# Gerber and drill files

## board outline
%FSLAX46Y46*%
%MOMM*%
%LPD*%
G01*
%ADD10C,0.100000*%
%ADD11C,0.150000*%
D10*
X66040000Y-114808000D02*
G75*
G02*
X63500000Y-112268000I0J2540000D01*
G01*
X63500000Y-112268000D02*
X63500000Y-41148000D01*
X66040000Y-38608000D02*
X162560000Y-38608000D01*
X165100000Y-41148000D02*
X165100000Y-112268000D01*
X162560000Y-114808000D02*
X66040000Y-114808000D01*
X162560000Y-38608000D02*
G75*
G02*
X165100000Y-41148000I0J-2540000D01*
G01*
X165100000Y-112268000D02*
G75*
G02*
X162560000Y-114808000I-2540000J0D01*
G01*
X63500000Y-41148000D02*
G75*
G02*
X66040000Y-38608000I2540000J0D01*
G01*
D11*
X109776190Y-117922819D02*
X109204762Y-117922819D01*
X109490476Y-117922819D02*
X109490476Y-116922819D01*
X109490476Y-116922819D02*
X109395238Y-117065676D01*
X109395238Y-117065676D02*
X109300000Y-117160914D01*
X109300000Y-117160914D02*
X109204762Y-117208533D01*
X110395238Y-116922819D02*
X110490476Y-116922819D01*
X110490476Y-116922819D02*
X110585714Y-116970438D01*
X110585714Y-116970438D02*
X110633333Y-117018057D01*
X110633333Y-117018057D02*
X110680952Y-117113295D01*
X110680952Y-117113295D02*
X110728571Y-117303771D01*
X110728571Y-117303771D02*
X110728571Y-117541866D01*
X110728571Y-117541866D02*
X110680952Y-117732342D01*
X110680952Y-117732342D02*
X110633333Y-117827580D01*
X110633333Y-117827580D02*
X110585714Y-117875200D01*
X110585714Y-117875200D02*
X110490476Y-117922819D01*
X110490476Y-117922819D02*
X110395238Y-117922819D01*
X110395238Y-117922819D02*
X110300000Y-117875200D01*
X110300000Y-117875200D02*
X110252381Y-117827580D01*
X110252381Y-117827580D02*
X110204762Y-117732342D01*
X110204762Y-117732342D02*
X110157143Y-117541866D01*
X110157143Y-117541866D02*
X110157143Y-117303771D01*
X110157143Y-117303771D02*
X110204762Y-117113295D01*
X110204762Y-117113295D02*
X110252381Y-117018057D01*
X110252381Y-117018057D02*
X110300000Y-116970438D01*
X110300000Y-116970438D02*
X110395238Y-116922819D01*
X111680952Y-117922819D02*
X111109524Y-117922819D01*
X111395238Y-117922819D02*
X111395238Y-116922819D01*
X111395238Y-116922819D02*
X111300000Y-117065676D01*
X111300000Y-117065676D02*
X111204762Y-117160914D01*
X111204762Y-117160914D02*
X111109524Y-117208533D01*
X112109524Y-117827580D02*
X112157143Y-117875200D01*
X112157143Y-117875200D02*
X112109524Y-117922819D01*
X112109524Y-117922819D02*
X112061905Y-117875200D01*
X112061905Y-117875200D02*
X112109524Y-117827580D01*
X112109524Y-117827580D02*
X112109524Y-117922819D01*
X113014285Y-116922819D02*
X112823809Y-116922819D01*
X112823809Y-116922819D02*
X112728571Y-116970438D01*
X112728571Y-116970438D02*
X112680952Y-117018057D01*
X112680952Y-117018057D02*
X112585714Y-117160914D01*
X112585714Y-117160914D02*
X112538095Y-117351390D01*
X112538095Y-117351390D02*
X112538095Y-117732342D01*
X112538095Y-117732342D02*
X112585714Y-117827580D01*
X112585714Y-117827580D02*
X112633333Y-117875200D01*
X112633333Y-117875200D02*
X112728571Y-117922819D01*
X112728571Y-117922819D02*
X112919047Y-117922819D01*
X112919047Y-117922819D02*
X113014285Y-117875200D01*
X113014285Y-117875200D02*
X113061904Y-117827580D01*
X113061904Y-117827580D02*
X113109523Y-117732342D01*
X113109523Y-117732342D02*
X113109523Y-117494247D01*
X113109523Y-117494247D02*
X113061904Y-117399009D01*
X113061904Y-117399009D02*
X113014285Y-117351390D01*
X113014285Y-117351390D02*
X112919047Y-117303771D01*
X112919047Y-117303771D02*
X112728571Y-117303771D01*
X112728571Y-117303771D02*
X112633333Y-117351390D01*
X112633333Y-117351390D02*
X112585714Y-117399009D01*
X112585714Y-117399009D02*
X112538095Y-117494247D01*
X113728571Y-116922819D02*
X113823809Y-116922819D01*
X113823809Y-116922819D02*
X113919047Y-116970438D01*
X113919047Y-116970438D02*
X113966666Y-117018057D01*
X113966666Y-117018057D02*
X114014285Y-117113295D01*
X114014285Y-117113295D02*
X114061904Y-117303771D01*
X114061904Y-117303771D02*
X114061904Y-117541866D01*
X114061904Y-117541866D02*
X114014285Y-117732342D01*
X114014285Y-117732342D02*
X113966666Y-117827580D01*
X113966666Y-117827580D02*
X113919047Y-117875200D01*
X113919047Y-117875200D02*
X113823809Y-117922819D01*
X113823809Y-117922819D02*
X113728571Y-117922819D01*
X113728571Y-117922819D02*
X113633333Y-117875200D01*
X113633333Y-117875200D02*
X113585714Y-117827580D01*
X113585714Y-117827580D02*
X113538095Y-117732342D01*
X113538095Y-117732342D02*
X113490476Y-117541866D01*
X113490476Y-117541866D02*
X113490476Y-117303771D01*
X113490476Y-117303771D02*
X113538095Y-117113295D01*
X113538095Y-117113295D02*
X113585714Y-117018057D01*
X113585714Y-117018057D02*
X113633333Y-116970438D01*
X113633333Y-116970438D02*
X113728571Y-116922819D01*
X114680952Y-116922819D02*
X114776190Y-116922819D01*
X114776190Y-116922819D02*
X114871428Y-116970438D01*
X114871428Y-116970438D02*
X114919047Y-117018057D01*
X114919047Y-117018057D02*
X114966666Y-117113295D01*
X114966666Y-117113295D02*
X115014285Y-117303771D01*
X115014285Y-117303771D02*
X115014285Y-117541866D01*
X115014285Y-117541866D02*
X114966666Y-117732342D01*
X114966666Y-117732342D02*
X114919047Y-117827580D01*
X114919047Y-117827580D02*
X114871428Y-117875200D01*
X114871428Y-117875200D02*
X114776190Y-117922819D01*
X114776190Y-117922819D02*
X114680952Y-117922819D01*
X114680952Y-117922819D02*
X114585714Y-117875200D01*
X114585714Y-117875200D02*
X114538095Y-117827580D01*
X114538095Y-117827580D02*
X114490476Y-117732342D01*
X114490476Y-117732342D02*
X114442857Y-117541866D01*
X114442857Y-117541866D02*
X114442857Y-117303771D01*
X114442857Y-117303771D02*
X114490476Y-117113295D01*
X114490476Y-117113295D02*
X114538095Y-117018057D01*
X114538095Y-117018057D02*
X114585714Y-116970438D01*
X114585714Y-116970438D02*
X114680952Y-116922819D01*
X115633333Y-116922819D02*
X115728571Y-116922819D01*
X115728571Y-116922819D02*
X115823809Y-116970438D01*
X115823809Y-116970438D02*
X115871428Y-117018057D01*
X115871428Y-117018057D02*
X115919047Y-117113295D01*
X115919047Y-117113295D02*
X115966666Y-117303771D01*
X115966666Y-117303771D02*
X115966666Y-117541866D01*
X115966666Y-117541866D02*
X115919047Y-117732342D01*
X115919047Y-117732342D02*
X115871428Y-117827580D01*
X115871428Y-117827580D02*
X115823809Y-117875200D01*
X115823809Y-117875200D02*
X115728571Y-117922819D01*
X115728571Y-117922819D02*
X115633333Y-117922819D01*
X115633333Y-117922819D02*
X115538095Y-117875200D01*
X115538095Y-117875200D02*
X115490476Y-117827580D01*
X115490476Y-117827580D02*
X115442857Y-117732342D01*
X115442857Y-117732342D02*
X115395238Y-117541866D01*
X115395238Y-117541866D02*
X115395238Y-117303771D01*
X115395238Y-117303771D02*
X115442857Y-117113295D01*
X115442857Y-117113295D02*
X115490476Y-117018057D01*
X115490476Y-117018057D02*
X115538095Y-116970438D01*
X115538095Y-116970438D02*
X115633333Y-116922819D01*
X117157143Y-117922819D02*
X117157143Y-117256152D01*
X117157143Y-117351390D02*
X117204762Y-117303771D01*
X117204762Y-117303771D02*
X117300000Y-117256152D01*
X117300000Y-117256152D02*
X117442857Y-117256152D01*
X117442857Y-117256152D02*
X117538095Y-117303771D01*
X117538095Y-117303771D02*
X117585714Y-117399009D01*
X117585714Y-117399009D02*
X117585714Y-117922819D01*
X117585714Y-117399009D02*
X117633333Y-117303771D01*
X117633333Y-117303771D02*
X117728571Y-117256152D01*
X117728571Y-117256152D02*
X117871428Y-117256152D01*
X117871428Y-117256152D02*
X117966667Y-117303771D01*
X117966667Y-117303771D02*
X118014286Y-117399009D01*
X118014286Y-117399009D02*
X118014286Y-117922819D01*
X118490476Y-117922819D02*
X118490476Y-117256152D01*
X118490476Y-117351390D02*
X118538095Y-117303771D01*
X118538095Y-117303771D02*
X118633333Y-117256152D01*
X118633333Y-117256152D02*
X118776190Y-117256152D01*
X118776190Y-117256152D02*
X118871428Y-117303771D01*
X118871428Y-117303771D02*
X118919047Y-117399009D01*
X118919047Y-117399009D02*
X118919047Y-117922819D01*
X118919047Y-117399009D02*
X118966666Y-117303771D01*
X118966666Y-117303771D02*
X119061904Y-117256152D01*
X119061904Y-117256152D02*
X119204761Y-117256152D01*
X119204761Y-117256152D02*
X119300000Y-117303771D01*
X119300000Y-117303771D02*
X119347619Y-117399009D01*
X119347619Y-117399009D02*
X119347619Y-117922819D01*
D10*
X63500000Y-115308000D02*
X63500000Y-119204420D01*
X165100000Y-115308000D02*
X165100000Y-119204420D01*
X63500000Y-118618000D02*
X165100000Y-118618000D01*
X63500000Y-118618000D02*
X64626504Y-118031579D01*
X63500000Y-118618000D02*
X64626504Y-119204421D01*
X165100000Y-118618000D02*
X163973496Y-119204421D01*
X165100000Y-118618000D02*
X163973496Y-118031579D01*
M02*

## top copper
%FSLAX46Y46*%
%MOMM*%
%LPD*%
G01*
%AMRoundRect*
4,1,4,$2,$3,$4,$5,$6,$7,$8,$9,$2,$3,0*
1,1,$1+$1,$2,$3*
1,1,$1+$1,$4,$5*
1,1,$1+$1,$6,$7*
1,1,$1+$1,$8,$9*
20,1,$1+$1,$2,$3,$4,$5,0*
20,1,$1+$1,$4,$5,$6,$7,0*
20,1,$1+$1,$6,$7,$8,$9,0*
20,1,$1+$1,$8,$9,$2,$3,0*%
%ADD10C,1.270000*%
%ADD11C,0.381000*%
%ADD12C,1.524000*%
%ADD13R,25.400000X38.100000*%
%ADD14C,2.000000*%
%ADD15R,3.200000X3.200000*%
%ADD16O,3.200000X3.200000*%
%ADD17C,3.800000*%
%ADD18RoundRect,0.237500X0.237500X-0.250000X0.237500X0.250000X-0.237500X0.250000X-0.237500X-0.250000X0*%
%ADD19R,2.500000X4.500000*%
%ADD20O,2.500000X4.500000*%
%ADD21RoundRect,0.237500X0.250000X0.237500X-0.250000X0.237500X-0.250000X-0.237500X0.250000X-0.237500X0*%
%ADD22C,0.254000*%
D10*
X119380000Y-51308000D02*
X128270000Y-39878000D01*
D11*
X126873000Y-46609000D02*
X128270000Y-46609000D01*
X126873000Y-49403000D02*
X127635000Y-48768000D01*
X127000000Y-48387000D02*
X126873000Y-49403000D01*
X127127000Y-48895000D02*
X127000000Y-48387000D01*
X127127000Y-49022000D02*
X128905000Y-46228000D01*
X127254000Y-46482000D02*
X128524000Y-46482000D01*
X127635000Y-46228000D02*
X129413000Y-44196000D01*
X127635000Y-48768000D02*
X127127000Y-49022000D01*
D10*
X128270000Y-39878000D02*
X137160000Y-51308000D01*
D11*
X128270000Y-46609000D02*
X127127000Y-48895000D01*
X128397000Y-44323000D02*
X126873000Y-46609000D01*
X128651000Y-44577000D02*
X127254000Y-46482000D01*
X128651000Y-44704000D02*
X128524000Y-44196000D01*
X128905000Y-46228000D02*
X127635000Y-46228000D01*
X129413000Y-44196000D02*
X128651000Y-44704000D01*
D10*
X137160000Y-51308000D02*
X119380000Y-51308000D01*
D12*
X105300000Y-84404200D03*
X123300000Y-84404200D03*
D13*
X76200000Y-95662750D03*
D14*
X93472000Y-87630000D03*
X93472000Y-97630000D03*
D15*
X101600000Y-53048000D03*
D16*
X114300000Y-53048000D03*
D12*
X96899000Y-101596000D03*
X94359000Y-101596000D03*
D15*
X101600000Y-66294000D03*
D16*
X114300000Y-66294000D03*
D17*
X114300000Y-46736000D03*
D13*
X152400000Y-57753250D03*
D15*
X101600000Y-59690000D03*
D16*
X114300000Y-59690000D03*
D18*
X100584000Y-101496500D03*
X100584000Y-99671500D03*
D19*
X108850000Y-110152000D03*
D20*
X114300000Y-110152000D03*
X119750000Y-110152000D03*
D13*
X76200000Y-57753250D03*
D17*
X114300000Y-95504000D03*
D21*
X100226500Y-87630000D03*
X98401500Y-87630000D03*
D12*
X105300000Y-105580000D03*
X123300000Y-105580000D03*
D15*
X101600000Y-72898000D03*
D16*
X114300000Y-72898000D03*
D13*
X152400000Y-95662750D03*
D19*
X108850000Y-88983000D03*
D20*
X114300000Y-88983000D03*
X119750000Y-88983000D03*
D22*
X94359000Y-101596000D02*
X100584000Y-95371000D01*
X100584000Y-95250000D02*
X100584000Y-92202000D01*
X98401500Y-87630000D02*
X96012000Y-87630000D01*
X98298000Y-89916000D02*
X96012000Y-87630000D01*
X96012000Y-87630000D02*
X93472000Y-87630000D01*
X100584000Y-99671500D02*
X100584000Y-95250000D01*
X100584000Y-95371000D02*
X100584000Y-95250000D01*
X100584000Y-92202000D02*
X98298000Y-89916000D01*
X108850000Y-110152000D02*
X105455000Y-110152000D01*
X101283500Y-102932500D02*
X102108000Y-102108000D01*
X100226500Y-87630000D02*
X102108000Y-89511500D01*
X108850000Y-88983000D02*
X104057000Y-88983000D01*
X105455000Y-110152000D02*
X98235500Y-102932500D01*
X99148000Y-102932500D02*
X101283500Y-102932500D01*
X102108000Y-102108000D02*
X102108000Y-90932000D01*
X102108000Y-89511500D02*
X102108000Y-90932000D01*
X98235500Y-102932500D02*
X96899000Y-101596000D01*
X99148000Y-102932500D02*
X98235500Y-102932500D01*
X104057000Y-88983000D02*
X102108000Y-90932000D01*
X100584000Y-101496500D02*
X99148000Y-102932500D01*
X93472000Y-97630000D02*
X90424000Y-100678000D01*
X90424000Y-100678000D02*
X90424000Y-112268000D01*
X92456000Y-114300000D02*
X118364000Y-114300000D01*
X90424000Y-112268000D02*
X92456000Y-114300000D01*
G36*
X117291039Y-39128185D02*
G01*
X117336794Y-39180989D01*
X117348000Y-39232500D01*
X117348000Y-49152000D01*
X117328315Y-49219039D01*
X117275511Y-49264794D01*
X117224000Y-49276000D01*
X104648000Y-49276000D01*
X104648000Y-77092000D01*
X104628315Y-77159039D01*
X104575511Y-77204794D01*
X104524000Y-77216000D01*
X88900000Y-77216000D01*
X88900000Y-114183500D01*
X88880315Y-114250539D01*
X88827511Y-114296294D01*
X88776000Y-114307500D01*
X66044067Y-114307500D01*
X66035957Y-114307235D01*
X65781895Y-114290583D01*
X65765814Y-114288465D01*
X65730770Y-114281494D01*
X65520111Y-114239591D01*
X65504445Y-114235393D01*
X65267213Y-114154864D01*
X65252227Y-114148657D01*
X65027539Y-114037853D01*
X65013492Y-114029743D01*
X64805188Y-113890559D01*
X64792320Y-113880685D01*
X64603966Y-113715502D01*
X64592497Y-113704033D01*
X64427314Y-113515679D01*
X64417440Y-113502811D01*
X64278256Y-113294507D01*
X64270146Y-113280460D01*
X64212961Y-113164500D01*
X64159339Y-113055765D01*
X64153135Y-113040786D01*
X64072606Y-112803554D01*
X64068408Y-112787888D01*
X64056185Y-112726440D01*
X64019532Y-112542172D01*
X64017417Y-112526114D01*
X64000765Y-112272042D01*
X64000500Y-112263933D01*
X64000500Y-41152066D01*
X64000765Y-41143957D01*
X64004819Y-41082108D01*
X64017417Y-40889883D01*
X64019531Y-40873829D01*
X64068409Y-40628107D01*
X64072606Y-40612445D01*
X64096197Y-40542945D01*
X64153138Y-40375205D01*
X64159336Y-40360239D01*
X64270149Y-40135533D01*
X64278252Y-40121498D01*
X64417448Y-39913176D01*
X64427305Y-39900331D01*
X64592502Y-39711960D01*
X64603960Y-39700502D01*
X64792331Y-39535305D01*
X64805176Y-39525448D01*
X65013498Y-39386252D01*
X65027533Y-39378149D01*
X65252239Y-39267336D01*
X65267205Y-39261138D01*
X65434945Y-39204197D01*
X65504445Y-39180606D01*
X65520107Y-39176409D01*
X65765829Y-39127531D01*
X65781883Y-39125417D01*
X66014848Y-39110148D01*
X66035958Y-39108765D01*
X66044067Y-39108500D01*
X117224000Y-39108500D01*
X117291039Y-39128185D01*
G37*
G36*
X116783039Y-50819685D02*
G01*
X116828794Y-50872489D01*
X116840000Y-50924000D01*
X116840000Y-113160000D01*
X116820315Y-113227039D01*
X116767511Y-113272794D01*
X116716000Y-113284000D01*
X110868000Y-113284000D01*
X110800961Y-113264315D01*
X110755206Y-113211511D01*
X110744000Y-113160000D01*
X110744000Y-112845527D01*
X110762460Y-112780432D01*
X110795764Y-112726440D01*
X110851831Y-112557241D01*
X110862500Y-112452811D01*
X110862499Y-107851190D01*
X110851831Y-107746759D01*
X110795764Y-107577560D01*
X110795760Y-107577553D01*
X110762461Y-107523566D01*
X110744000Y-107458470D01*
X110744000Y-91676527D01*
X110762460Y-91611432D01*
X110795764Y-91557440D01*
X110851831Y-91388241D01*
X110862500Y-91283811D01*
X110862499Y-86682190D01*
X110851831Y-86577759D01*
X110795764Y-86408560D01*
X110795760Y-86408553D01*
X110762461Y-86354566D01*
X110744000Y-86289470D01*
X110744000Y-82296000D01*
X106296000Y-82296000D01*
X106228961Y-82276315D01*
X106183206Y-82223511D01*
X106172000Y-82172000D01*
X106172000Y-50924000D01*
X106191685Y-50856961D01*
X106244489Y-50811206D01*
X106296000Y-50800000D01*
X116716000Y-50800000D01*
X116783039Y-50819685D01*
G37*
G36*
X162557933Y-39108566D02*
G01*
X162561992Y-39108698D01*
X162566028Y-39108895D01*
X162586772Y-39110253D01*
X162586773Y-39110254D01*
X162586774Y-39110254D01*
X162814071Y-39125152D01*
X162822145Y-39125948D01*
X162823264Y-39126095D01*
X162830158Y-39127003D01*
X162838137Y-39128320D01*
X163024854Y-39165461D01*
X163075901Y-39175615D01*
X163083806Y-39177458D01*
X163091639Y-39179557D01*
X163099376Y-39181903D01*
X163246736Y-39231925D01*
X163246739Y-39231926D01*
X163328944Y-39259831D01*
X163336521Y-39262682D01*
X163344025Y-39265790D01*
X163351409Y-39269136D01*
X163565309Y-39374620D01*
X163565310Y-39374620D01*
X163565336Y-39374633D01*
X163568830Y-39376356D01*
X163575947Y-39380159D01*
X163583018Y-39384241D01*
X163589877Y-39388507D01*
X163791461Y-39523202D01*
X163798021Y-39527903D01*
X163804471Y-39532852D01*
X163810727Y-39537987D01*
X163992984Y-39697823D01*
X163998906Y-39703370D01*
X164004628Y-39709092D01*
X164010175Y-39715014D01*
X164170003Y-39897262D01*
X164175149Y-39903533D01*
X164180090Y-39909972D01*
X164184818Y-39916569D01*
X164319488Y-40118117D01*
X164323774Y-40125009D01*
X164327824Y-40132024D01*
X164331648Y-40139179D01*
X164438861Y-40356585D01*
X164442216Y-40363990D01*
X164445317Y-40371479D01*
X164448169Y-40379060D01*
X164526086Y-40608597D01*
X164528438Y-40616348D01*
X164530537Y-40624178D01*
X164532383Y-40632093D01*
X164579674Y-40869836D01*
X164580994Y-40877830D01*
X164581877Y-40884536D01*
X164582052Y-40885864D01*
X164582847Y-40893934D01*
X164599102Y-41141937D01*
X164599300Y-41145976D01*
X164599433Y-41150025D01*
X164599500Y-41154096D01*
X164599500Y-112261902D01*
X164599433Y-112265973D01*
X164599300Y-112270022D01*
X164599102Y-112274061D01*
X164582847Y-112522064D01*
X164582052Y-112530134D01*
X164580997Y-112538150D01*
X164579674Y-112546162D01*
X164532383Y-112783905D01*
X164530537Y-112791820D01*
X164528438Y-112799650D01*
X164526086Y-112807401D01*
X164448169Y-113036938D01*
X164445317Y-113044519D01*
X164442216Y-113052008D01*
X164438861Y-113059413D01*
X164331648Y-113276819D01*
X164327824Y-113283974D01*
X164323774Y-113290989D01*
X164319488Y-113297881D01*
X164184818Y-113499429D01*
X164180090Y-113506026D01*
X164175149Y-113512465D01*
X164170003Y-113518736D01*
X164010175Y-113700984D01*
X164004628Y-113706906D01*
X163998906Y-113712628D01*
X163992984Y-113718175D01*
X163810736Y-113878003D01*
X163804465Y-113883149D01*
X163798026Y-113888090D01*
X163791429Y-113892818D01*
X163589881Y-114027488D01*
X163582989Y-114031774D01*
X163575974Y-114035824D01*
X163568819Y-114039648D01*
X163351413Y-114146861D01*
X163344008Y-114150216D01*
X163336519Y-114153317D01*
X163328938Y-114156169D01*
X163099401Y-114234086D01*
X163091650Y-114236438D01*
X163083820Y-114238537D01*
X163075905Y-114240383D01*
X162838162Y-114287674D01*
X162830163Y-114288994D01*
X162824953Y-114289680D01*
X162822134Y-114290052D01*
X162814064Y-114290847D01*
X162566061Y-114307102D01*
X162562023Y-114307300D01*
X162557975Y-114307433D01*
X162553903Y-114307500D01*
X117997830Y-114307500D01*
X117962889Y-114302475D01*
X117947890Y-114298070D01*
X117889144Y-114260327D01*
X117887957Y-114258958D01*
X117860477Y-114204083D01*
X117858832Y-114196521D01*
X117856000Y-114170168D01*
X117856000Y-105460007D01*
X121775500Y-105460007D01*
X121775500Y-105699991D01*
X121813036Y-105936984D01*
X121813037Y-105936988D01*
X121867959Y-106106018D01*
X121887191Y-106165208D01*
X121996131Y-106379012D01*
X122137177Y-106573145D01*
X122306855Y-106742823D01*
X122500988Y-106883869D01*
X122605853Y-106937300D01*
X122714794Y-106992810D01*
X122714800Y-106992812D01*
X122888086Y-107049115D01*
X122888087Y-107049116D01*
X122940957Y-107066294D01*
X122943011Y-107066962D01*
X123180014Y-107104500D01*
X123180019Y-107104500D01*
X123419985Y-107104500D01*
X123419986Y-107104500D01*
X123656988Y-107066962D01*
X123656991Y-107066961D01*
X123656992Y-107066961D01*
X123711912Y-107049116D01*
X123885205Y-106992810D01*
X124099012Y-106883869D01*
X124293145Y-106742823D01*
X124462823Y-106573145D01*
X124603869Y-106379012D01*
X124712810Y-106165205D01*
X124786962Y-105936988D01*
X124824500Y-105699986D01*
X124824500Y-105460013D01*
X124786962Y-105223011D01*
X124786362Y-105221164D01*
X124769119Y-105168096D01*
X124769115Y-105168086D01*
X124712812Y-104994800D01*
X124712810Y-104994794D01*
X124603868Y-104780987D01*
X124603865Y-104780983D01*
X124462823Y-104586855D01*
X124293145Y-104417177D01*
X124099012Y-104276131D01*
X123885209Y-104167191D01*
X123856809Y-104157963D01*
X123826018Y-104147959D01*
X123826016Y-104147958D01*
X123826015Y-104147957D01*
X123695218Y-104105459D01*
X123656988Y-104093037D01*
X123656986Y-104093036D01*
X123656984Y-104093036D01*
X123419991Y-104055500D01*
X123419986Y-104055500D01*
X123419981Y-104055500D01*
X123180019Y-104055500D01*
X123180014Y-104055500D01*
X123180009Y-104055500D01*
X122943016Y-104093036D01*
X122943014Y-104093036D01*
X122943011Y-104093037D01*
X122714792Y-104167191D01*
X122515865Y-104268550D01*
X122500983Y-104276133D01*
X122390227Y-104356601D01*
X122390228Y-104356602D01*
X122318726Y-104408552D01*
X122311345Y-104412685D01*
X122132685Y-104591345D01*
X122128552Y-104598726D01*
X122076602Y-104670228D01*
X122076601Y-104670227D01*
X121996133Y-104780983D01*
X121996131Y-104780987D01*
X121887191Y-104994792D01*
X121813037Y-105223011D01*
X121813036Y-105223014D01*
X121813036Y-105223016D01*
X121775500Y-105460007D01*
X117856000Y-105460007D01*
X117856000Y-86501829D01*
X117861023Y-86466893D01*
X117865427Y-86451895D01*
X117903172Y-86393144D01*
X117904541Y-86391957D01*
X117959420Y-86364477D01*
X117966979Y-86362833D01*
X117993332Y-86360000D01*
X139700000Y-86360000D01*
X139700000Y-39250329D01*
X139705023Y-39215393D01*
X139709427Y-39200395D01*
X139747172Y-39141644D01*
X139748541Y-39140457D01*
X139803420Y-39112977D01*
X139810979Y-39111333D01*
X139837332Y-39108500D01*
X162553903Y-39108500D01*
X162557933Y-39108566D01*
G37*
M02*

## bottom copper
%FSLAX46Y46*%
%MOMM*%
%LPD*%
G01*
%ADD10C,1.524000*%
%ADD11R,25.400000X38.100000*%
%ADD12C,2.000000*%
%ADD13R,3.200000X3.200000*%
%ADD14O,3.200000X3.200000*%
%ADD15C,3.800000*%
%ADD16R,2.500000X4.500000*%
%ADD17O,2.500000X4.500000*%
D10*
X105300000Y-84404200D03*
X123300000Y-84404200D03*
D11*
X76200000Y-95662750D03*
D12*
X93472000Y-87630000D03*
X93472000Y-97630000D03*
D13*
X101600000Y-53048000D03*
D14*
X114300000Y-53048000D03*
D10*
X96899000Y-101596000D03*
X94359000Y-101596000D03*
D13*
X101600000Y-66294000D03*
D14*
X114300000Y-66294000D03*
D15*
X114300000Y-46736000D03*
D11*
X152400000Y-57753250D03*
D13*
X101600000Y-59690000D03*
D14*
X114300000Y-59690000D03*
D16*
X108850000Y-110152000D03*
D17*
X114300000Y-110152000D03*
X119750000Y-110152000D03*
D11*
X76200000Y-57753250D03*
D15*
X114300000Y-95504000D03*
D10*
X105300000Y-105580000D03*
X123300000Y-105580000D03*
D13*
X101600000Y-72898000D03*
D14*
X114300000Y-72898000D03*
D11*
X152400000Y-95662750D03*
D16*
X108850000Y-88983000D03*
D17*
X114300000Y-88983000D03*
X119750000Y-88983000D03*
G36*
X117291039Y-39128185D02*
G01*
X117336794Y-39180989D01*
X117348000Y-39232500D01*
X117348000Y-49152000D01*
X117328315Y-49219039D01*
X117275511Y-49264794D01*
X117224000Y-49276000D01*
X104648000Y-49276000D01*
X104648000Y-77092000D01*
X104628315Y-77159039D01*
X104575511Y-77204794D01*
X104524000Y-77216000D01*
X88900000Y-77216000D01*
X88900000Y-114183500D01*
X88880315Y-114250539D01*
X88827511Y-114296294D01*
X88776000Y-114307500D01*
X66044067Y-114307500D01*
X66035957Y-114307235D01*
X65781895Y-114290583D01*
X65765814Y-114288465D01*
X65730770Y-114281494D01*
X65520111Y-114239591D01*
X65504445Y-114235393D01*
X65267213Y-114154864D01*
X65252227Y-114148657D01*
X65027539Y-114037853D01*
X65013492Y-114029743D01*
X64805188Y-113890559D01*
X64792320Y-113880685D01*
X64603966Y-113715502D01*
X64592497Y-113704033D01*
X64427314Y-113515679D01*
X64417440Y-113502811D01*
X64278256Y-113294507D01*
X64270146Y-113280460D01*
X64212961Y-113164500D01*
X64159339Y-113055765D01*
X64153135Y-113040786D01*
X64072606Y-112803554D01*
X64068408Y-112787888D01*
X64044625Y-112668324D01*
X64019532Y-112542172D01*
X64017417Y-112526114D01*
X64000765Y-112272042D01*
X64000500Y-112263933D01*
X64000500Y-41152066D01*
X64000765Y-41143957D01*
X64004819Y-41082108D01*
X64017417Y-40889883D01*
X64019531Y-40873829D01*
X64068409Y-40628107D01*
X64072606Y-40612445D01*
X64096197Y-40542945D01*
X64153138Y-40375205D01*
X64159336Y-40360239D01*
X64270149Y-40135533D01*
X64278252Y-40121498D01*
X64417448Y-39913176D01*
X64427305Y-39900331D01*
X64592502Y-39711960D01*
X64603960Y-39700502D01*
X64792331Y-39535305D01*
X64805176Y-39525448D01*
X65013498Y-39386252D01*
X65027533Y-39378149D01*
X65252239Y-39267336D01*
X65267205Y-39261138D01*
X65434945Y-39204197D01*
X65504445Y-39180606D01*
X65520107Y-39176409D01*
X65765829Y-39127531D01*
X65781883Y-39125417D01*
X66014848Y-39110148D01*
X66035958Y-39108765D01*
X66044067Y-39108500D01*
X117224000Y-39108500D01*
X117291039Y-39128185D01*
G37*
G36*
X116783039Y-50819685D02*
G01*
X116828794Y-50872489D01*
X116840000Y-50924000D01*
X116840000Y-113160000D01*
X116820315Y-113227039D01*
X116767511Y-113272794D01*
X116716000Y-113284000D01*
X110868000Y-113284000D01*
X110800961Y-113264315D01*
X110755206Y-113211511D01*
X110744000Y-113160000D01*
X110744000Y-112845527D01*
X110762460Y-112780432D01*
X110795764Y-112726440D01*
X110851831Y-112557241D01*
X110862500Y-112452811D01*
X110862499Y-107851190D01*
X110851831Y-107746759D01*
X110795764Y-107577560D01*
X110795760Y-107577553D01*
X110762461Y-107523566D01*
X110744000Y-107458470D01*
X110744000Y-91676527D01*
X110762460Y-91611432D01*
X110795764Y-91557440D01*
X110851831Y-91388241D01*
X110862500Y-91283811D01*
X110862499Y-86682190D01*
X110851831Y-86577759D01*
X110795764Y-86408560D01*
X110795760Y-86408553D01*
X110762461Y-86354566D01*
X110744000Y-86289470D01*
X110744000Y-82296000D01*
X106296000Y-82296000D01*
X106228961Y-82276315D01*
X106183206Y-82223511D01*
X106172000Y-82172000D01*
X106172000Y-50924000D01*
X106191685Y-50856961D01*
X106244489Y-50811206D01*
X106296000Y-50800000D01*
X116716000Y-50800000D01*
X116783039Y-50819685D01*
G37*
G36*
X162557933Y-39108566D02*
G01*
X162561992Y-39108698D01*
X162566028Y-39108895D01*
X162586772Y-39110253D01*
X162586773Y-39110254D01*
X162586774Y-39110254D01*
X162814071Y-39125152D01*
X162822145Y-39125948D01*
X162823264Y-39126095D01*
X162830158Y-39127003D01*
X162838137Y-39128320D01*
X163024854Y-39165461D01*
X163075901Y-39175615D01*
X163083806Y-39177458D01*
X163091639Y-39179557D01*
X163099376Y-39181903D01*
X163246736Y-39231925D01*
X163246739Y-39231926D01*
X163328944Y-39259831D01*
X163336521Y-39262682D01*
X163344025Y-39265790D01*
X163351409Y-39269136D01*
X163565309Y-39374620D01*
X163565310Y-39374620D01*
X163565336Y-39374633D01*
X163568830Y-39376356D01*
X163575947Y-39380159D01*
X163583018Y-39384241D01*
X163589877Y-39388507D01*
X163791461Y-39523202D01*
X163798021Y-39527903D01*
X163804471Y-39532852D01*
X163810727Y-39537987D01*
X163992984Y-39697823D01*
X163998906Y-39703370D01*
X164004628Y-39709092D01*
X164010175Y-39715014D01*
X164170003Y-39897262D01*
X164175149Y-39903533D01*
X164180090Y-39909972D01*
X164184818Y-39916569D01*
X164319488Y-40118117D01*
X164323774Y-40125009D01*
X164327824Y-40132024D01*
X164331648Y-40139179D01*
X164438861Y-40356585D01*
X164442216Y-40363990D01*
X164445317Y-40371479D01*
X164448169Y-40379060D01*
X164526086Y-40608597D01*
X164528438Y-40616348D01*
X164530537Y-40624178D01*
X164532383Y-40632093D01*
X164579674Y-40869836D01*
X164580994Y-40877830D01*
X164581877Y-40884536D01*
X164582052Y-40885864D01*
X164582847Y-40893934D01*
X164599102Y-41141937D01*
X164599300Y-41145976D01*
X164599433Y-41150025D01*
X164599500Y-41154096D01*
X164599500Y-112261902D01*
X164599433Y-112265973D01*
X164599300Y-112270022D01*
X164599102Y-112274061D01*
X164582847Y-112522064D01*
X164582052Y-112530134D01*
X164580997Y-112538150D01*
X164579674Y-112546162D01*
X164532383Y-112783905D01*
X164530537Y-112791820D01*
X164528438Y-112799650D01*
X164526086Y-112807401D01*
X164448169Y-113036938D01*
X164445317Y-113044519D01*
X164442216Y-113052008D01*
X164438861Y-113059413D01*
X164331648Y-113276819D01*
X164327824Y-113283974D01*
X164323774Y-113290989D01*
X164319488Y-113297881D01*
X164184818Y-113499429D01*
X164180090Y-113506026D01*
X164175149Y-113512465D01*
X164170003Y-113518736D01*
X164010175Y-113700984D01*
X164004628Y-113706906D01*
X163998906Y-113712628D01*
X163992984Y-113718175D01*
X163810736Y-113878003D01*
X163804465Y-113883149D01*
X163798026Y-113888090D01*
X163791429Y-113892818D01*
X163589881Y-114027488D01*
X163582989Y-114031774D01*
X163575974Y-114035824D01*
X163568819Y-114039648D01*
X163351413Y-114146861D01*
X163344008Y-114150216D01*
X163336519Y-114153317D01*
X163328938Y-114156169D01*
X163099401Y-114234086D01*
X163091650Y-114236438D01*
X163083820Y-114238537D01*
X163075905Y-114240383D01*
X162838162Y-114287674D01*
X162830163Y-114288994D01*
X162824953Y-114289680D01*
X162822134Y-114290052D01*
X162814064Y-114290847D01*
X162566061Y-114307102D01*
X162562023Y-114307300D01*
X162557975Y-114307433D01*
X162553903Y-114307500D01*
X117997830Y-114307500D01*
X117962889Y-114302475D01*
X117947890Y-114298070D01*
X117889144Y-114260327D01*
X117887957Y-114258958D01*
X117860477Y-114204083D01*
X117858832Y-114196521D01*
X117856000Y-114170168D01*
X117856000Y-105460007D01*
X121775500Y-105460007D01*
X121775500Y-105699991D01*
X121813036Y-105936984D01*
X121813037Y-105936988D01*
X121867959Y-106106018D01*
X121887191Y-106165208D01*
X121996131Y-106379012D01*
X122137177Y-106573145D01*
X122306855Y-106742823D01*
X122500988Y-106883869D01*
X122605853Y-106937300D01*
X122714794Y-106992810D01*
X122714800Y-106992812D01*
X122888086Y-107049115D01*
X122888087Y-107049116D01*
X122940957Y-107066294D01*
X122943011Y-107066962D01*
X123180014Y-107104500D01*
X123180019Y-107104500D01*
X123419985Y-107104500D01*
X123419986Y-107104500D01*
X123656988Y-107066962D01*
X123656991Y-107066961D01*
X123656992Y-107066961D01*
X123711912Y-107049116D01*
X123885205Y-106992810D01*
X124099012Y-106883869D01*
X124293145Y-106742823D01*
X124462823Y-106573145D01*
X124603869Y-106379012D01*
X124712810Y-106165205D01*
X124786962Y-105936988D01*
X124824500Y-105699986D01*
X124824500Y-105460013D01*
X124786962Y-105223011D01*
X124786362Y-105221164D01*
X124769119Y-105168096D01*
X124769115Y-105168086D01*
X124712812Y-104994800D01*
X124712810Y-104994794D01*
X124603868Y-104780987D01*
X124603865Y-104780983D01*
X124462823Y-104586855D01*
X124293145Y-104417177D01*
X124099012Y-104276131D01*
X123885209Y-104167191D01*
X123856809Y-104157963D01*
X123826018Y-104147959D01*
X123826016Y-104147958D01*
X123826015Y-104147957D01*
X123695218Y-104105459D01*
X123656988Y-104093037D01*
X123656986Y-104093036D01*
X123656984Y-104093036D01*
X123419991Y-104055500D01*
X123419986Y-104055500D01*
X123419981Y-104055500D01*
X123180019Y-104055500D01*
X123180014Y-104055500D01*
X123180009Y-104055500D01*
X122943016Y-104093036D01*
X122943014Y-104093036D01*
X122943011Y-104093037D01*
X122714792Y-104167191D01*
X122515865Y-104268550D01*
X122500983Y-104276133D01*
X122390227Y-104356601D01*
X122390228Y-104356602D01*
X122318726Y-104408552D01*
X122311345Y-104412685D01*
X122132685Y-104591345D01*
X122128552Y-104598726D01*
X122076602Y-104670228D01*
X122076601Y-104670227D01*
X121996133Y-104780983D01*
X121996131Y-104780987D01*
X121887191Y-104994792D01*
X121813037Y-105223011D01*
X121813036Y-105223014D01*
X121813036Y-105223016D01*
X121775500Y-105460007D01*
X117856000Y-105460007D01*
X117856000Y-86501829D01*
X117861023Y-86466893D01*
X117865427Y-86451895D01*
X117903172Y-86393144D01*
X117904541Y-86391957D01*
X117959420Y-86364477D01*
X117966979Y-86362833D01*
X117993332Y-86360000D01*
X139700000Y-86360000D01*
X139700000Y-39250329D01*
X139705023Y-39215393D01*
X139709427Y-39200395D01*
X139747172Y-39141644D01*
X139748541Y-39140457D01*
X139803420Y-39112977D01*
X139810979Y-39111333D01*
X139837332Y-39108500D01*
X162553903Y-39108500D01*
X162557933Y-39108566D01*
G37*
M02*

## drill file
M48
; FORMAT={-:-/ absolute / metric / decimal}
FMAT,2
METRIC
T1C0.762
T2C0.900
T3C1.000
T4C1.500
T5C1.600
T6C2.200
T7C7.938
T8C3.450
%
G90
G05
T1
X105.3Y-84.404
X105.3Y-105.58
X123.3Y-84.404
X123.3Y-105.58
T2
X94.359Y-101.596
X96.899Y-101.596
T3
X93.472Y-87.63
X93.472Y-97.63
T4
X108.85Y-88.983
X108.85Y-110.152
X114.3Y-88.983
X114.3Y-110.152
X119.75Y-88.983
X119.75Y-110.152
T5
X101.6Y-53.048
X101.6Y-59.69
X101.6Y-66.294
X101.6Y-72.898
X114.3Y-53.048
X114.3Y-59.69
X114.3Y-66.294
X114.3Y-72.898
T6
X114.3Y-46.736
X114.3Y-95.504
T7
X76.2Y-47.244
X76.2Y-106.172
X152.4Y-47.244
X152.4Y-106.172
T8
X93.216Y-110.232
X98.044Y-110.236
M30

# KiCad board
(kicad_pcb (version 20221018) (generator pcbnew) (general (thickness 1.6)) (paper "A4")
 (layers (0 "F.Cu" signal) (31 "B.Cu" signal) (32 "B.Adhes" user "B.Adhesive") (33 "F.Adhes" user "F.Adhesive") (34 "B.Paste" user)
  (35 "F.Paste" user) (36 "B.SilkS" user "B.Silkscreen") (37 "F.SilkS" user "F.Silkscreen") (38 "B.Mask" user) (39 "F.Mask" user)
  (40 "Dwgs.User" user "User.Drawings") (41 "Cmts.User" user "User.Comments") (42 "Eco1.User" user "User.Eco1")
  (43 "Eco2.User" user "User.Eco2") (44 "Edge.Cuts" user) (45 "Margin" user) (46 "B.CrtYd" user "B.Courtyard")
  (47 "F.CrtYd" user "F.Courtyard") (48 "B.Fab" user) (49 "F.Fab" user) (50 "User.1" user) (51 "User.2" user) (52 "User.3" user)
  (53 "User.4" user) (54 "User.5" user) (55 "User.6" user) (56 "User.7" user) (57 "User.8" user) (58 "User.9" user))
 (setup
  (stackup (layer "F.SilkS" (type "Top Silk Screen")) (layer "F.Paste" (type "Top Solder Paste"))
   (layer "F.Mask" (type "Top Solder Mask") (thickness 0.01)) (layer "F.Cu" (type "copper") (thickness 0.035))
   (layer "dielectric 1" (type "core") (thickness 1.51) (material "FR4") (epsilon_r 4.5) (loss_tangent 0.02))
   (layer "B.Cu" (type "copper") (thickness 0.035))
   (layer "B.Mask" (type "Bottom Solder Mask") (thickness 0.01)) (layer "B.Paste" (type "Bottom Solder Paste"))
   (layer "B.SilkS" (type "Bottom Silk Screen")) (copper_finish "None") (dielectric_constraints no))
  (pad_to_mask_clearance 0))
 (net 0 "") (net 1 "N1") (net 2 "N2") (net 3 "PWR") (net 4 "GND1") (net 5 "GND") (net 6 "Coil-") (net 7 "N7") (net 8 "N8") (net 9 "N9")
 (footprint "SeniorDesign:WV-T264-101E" (layer "F.Cu") (at 114.3 84.4042)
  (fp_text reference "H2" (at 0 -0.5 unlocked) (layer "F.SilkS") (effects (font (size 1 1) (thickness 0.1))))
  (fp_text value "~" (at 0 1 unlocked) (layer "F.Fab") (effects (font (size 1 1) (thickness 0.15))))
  (pad "1" thru_hole circle (at -9 0) (size 1.524 1.524) (drill 0.762) (layers "*.Cu" "*.Mask") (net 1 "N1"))
  (pad "2" thru_hole circle (at 9 0) (size 1.524 1.524) (drill 0.762) (layers "*.Cu" "*.Mask") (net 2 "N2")))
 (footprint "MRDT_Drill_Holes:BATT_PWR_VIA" (layer "F.Cu") (at 76.2 106.172)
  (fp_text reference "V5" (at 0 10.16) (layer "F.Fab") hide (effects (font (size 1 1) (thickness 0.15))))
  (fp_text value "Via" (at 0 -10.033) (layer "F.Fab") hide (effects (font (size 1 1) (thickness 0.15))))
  (pad "1" thru_hole rect (at 0 0) (size 25.4 38.1) (drill 7.9375 (offset 0 -10.50925)) (layers "*.Cu" "*.Mask") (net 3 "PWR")
   (zone_connect 2)))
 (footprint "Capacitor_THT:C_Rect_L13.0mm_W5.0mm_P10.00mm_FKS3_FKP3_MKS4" (layer "F.Cu") (at 93.472 87.63 -90)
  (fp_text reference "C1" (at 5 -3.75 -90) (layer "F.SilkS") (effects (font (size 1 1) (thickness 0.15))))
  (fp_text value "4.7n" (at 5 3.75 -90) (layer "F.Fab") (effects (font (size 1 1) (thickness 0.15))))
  (pad "1" thru_hole circle (at 0 0 270) (size 2 2) (drill 1) (layers "*.Cu" "*.Mask") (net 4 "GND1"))
  (pad "2" thru_hole circle (at 10 0 270) (size 2 2) (drill 1) (layers "*.Cu" "*.Mask") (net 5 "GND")))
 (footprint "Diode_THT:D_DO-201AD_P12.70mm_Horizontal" (layer "F.Cu") (at 101.6 53.048)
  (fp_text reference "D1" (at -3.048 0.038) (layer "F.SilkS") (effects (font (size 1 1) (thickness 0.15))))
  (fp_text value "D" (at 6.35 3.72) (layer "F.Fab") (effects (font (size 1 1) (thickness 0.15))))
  (pad "1" thru_hole rect (at 0 0) (size 3.2 3.2) (drill 1.6) (layers "*.Cu" "*.Mask") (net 3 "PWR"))
  (pad "2" thru_hole oval (at 12.7 0) (size 3.2 3.2) (drill 1.6) (layers "*.Cu" "*.Mask") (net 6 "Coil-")))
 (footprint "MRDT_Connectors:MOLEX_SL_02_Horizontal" (layer "F.Cu") (at 96.899 101.596 180)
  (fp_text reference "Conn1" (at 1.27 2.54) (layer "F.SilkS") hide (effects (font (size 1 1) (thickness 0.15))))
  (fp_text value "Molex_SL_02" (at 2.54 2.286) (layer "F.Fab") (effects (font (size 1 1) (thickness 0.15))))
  (pad "" np_thru_hole circle (at -1.145 -8.64 180) (size 3.45 3.45) (drill 3.45) (layers "*.Cu" "*.Mask"))
  (pad "" np_thru_hole circle (at 3.683 -8.636 180) (size 3.45 3.45) (drill 3.45) (layers "*.Cu" "*.Mask"))
  (pad "1" thru_hole circle (at 0 0 180) (size 1.524 1.524) (drill 0.9) (layers "*.Cu" "*.Mask") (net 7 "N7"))
  (pad "2" thru_hole circle (at 2.54 0 180) (size 1.524 1.524) (drill 0.9) (layers "*.Cu" "*.Mask") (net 4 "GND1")))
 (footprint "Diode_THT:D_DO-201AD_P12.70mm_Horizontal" (layer "F.Cu") (at 101.6 66.294)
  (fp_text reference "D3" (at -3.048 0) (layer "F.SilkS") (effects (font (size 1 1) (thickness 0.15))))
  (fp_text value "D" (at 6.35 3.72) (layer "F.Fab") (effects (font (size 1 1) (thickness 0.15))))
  (pad "1" thru_hole rect (at 0 0) (size 3.2 3.2) (drill 1.6) (layers "*.Cu" "*.Mask") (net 3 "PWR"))
  (pad "2" thru_hole oval (at 12.7 0) (size 3.2 3.2) (drill 1.6) (layers "*.Cu" "*.Mask") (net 6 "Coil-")))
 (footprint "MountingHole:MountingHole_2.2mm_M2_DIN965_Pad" (layer "F.Cu") (at 114.3 46.736)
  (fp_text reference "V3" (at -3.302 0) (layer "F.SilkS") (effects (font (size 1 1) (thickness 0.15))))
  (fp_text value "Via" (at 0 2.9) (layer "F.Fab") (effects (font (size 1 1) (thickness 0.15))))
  (pad "1" thru_hole circle (at 0 0) (size 3.8 3.8) (drill 2.2) (layers "*.Cu" "*.Mask") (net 3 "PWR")))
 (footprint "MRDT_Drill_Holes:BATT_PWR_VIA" (layer "F.Cu") (at 152.4 47.244)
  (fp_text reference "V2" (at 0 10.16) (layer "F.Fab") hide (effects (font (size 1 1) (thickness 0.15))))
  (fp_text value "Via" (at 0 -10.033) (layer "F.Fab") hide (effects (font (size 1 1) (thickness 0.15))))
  (pad "1" thru_hole rect (at 0 0) (size 25.4 38.1) (drill 7.9375 (offset 0 10.50925)) (layers "*.Cu" "*.Mask") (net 5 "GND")
   (zone_connect 2)))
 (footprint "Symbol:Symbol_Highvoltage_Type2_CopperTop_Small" (layer "F.Cu") (at 128.27 47.498)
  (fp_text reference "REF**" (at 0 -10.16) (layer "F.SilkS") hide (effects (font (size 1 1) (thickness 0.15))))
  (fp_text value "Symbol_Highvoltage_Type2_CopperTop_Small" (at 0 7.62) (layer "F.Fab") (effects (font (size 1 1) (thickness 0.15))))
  (fp_line (start -8.89 3.81) (end 0 -7.62) (stroke (width 1.27) (type solid)) (layer "F.Cu"))
  (fp_line (start -1.397 -0.889) (end 0 -0.889) (stroke (width 0.381) (type solid)) (layer "F.Cu"))
  (fp_line (start -1.397 1.905) (end -0.635 1.27) (stroke (width 0.381) (type solid)) (layer "F.Cu"))
  (fp_line (start -1.27 0.889) (end -1.397 1.905) (stroke (width 0.381) (type solid)) (layer "F.Cu"))
  (fp_line (start -1.143 1.397) (end -1.27 0.889) (stroke (width 0.381) (type solid)) (layer "F.Cu"))
  (fp_line (start -1.143 1.524) (end 0.635 -1.27) (stroke (width 0.381) (type solid)) (layer "F.Cu"))
  (fp_line (start -1.016 -1.016) (end 0.254 -1.016) (stroke (width 0.381) (type solid)) (layer "F.Cu"))
  (fp_line (start -0.635 -1.27) (end 1.143 -3.302) (stroke (width 0.381) (type solid)) (layer "F.Cu"))
  (fp_line (start -0.635 1.27) (end -1.143 1.524) (stroke (width 0.381) (type solid)) (layer "F.Cu"))
  (fp_line (start 0 -7.62) (end 8.89 3.81) (stroke (width 1.27) (type solid)) (layer "F.Cu"))
  (fp_line (start 0 -0.889) (end -1.143 1.397) (stroke (width 0.381) (type solid)) (layer "F.Cu"))
  (fp_line (start 0.127 -3.175) (end -1.397 -0.889) (stroke (width 0.381) (type solid)) (layer "F.Cu"))
  (fp_line (start 0.381 -2.921) (end -1.016 -1.016) (stroke (width 0.381) (type solid)) (layer "F.Cu"))
  (fp_line (start 0.381 -2.794) (end 0.254 -3.302) (stroke (width 0.381) (type solid)) (layer "F.Cu"))
  (fp_line (start 0.635 -1.27) (end -0.635 -1.27) (stroke (width 0.381) (type solid)) (layer "F.Cu"))
  (fp_line (start 1.143 -3.302) (end 0.381 -2.794) (stroke (width 0.381) (type solid)) (layer "F.Cu"))
  (fp_line (start 8.89 3.81) (end -8.89 3.81) (stroke (width 1.27) (type solid)) (layer "F.Cu")))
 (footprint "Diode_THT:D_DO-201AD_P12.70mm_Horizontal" (layer "F.Cu") (at 101.6 59.69)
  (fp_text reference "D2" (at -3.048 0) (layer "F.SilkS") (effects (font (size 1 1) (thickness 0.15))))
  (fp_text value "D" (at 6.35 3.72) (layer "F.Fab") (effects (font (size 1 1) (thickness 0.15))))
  (pad "1" thru_hole rect (at 0 0) (size 3.2 3.2) (drill 1.6) (layers "*.Cu" "*.Mask") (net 3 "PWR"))
  (pad "2" thru_hole oval (at 12.7 0) (size 3.2 3.2) (drill 1.6) (layers "*.Cu" "*.Mask") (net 6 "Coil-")))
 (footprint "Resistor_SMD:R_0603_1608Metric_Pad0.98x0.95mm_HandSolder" (layer "F.Cu") (at 100.584 100.584 90)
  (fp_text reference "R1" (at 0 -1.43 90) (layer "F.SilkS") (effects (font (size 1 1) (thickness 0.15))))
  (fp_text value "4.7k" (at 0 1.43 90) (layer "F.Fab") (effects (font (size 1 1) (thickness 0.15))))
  (pad "1" smd roundrect (at -0.9125 0 90) (size 0.975 0.95) (layers "F.Cu" "F.Paste" "F.Mask") (roundrect_rratio 0.25) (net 7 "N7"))
  (pad "2" smd roundrect (at 0.9125 0 90) (size 0.975 0.95) (layers "F.Cu" "F.Paste" "F.Mask") (roundrect_rratio 0.25) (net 4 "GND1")))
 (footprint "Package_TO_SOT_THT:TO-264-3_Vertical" (layer "F.Cu") (at 108.85 110.152)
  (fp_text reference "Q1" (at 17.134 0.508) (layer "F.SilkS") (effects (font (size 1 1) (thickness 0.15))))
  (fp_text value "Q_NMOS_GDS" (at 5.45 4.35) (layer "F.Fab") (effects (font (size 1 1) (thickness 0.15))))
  (pad "1" thru_hole rect (at 0 0) (size 2.5 4.5) (drill 1.5) (layers "*.Cu" "*.Mask") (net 7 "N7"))
  (pad "2" thru_hole oval (at 5.45 0) (size 2.5 4.5) (drill 1.5) (layers "*.Cu" "*.Mask") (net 6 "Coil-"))
  (pad "3" thru_hole oval (at 10.9 0) (size 2.5 4.5) (drill 1.5) (layers "*.Cu" "*.Mask") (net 5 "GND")))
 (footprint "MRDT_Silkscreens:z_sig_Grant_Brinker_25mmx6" (layer "F.Cu") (at 125.73 60.706 45)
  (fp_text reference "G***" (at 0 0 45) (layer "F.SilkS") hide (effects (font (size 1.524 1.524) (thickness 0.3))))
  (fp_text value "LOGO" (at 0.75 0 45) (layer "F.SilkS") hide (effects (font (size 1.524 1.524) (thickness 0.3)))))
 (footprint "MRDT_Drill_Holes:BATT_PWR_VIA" (layer "F.Cu") (at 76.2 47.244)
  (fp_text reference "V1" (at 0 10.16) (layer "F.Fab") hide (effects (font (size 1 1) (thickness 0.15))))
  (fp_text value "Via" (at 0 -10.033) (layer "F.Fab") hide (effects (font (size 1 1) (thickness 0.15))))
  (pad "1" thru_hole rect (at 0 0) (size 25.4 38.1) (drill 7.9375 (offset 0 10.50925)) (layers "*.Cu" "*.Mask") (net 3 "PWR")
   (zone_connect 2)))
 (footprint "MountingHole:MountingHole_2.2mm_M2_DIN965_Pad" (layer "F.Cu") (at 114.3 95.504)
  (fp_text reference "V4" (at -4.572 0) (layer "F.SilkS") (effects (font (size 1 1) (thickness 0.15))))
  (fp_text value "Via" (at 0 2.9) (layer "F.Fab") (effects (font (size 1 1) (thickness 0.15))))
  (pad "1" thru_hole circle (at 0 0) (size 3.8 3.8) (drill 2.2) (layers "*.Cu" "*.Mask") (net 6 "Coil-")))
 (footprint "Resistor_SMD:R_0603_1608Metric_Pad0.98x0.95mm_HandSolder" (layer "F.Cu") (at 99.314 87.63 180)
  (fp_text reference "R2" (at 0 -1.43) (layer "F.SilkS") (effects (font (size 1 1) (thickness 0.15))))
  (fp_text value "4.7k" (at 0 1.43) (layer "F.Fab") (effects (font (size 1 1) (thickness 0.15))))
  (pad "1" smd roundrect (at -0.9125 0 180) (size 0.975 0.95) (layers "F.Cu" "F.Paste" "F.Mask") (roundrect_rratio 0.25) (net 7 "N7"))
  (pad "2" smd roundrect (at 0.9125 0 180) (size 0.975 0.95) (layers "F.Cu" "F.Paste" "F.Mask") (roundrect_rratio 0.25) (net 4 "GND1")))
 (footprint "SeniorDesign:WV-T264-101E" (layer "F.Cu") (at 114.3 105.58)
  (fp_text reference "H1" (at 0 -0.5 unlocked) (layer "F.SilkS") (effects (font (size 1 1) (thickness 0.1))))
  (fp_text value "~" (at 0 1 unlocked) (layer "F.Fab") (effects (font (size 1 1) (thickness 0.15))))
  (pad "1" thru_hole circle (at -9 0) (size 1.524 1.524) (drill 0.762) (layers "*.Cu" "*.Mask") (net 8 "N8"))
  (pad "2" thru_hole circle (at 9 0) (size 1.524 1.524) (drill 0.762) (layers "*.Cu" "*.Mask") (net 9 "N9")))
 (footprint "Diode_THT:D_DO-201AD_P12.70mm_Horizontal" (layer "F.Cu") (at 101.6 72.898)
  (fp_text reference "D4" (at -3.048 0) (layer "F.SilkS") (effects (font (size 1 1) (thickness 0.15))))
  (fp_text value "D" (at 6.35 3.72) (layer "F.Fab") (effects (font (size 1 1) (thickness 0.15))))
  (pad "1" thru_hole rect (at 0 0) (size 3.2 3.2) (drill 1.6) (layers "*.Cu" "*.Mask") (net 3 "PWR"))
  (pad "2" thru_hole oval (at 12.7 0) (size 3.2 3.2) (drill 1.6) (layers "*.Cu" "*.Mask") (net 6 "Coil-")))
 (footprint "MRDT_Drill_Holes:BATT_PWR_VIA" (layer "F.Cu") (at 152.4 106.172)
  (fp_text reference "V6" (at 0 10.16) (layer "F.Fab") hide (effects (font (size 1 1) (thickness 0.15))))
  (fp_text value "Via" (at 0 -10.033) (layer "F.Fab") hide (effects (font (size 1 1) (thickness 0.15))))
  (pad "1" thru_hole rect (at 0 0) (size 25.4 38.1) (drill 7.9375 (offset 0 -10.50925)) (layers "*.Cu" "*.Mask") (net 5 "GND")
   (zone_connect 2)))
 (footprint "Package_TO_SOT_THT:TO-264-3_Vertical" (layer "F.Cu") (at 108.85 88.983)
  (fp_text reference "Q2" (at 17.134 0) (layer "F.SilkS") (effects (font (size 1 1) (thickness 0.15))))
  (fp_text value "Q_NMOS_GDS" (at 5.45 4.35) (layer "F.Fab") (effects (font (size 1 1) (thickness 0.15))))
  (pad "1" thru_hole rect (at 0 0) (size 2.5 4.5) (drill 1.5) (layers "*.Cu" "*.Mask") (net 7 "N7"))
  (pad "2" thru_hole oval (at 5.45 0) (size 2.5 4.5) (drill 1.5) (layers "*.Cu" "*.Mask") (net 6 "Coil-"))
  (pad "3" thru_hole oval (at 10.9 0) (size 2.5 4.5) (drill 1.5) (layers "*.Cu" "*.Mask") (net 5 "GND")))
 (gr_arc (start 66.04 114.808) (mid 64.243949 114.064051) (end 63.5 112.268) (stroke (width 0.1) (type default)) (layer "Edge.Cuts"))
 (gr_line (start 63.5 112.268) (end 63.5 41.148) (stroke (width 0.1) (type default)) (layer "Edge.Cuts"))
 (gr_line (start 66.04 38.608) (end 162.56 38.608) (stroke (width 0.1) (type default)) (layer "Edge.Cuts"))
 (gr_line (start 165.1 41.148) (end 165.1 112.268) (stroke (width 0.1) (type default)) (layer "Edge.Cuts"))
 (gr_line (start 162.56 114.808) (end 66.04 114.808) (stroke (width 0.1) (type default)) (layer "Edge.Cuts"))
 (gr_arc (start 162.56 38.608) (mid 164.356051 39.351949) (end 165.1 41.148) (stroke (width 0.1) (type default)) (layer "Edge.Cuts"))
 (gr_arc (start 165.1 112.268) (mid 164.356051 114.064051) (end 162.56 114.808) (stroke (width 0.1) (type default)) (layer "Edge.Cuts"))
 (gr_arc (start 63.5 41.148) (mid 64.243949 39.351949) (end 66.04 38.608) (stroke (width 0.1) (type default)) (layer "Edge.Cuts"))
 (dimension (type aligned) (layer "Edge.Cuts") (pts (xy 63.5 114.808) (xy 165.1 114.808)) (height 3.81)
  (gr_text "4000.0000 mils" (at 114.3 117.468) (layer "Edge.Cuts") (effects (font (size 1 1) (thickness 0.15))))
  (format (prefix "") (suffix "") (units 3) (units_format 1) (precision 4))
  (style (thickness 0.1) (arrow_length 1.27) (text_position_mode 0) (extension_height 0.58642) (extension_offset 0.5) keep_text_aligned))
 (segment (start 94.359 101.596) (end 100.584 95.371) (width 0.254) (layer "F.Cu") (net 4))
 (segment (start 100.584 95.25) (end 100.584 92.202) (width 0.254) (layer "F.Cu") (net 4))
 (segment (start 98.4015 87.63) (end 96.012 87.63) (width 0.254) (layer "F.Cu") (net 4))
 (segment (start 98.298 89.916) (end 96.012 87.63) (width 0.254) (layer "F.Cu") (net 4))
 (segment (start 96.012 87.63) (end 93.472 87.63) (width 0.254) (layer "F.Cu") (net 4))
 (segment (start 100.584 99.6715) (end 100.584 95.25) (width 0.254) (layer "F.Cu") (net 4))
 (segment (start 100.584 95.371) (end 100.584 95.25) (width 0.254) (layer "F.Cu") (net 4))
 (segment (start 100.584 92.202) (end 98.298 89.916) (width 0.254) (layer "F.Cu") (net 4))
 (segment (start 108.85 110.152) (end 105.455 110.152) (width 0.254) (layer "F.Cu") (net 7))
 (segment (start 101.2835 102.9325) (end 102.108 102.108) (width 0.254) (layer "F.Cu") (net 7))
 (segment (start 100.2265 87.63) (end 102.108 89.5115) (width 0.254) (layer "F.Cu") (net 7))
 (segment (start 108.85 88.983) (end 104.057 88.983) (width 0.254) (layer "F.Cu") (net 7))
 (segment (start 105.455 110.152) (end 98.2355 102.9325) (width 0.254) (layer "F.Cu") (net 7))
 (segment (start 99.148 102.9325) (end 101.2835 102.9325) (width 0.254) (layer "F.Cu") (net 7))
 (segment (start 102.108 102.108) (end 102.108 90.932) (width 0.254) (layer "F.Cu") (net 7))
 (segment (start 102.108 89.5115) (end 102.108 90.932) (width 0.254) (layer "F.Cu") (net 7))
 (segment (start 98.2355 102.9325) (end 96.899 101.596) (width 0.254) (layer "F.Cu") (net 7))
 (segment (start 99.148 102.9325) (end 98.2355 102.9325) (width 0.254) (layer "F.Cu") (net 7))
 (segment (start 104.057 88.983) (end 102.108 90.932) (width 0.254) (layer "F.Cu") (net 7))
 (segment (start 100.584 101.4965) (end 99.148 102.9325) (width 0.254) (layer "F.Cu") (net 7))
 (segment (start 93.472 97.63) (end 90.424 100.678) (width 0.254) (layer "F.Cu") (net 5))
 (segment (start 90.424 100.678) (end 90.424 112.268) (width 0.254) (layer "F.Cu") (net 5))
 (segment (start 92.456 114.3) (end 118.364 114.3) (width 0.254) (layer "F.Cu") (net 5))
 (segment (start 90.424 112.268) (end 92.456 114.3) (width 0.254) (layer "F.Cu") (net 5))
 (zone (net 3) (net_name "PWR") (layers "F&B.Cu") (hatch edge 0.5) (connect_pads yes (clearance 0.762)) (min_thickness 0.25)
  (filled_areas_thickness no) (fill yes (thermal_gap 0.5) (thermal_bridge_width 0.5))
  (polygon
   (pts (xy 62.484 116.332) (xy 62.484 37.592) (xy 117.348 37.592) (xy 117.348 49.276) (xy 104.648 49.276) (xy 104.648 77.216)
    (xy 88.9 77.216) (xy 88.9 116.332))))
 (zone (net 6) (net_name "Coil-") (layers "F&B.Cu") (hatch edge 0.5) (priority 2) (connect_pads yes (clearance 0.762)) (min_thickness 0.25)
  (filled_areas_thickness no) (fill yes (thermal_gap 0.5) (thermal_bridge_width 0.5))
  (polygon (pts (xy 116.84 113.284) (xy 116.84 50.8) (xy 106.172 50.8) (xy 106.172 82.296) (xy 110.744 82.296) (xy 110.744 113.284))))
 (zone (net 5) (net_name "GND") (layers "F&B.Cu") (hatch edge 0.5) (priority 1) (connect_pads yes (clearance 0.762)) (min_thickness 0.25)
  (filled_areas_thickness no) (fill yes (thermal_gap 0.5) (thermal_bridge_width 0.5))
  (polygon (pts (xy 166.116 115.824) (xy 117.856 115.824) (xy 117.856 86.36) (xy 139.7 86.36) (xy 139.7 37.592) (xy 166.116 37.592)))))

